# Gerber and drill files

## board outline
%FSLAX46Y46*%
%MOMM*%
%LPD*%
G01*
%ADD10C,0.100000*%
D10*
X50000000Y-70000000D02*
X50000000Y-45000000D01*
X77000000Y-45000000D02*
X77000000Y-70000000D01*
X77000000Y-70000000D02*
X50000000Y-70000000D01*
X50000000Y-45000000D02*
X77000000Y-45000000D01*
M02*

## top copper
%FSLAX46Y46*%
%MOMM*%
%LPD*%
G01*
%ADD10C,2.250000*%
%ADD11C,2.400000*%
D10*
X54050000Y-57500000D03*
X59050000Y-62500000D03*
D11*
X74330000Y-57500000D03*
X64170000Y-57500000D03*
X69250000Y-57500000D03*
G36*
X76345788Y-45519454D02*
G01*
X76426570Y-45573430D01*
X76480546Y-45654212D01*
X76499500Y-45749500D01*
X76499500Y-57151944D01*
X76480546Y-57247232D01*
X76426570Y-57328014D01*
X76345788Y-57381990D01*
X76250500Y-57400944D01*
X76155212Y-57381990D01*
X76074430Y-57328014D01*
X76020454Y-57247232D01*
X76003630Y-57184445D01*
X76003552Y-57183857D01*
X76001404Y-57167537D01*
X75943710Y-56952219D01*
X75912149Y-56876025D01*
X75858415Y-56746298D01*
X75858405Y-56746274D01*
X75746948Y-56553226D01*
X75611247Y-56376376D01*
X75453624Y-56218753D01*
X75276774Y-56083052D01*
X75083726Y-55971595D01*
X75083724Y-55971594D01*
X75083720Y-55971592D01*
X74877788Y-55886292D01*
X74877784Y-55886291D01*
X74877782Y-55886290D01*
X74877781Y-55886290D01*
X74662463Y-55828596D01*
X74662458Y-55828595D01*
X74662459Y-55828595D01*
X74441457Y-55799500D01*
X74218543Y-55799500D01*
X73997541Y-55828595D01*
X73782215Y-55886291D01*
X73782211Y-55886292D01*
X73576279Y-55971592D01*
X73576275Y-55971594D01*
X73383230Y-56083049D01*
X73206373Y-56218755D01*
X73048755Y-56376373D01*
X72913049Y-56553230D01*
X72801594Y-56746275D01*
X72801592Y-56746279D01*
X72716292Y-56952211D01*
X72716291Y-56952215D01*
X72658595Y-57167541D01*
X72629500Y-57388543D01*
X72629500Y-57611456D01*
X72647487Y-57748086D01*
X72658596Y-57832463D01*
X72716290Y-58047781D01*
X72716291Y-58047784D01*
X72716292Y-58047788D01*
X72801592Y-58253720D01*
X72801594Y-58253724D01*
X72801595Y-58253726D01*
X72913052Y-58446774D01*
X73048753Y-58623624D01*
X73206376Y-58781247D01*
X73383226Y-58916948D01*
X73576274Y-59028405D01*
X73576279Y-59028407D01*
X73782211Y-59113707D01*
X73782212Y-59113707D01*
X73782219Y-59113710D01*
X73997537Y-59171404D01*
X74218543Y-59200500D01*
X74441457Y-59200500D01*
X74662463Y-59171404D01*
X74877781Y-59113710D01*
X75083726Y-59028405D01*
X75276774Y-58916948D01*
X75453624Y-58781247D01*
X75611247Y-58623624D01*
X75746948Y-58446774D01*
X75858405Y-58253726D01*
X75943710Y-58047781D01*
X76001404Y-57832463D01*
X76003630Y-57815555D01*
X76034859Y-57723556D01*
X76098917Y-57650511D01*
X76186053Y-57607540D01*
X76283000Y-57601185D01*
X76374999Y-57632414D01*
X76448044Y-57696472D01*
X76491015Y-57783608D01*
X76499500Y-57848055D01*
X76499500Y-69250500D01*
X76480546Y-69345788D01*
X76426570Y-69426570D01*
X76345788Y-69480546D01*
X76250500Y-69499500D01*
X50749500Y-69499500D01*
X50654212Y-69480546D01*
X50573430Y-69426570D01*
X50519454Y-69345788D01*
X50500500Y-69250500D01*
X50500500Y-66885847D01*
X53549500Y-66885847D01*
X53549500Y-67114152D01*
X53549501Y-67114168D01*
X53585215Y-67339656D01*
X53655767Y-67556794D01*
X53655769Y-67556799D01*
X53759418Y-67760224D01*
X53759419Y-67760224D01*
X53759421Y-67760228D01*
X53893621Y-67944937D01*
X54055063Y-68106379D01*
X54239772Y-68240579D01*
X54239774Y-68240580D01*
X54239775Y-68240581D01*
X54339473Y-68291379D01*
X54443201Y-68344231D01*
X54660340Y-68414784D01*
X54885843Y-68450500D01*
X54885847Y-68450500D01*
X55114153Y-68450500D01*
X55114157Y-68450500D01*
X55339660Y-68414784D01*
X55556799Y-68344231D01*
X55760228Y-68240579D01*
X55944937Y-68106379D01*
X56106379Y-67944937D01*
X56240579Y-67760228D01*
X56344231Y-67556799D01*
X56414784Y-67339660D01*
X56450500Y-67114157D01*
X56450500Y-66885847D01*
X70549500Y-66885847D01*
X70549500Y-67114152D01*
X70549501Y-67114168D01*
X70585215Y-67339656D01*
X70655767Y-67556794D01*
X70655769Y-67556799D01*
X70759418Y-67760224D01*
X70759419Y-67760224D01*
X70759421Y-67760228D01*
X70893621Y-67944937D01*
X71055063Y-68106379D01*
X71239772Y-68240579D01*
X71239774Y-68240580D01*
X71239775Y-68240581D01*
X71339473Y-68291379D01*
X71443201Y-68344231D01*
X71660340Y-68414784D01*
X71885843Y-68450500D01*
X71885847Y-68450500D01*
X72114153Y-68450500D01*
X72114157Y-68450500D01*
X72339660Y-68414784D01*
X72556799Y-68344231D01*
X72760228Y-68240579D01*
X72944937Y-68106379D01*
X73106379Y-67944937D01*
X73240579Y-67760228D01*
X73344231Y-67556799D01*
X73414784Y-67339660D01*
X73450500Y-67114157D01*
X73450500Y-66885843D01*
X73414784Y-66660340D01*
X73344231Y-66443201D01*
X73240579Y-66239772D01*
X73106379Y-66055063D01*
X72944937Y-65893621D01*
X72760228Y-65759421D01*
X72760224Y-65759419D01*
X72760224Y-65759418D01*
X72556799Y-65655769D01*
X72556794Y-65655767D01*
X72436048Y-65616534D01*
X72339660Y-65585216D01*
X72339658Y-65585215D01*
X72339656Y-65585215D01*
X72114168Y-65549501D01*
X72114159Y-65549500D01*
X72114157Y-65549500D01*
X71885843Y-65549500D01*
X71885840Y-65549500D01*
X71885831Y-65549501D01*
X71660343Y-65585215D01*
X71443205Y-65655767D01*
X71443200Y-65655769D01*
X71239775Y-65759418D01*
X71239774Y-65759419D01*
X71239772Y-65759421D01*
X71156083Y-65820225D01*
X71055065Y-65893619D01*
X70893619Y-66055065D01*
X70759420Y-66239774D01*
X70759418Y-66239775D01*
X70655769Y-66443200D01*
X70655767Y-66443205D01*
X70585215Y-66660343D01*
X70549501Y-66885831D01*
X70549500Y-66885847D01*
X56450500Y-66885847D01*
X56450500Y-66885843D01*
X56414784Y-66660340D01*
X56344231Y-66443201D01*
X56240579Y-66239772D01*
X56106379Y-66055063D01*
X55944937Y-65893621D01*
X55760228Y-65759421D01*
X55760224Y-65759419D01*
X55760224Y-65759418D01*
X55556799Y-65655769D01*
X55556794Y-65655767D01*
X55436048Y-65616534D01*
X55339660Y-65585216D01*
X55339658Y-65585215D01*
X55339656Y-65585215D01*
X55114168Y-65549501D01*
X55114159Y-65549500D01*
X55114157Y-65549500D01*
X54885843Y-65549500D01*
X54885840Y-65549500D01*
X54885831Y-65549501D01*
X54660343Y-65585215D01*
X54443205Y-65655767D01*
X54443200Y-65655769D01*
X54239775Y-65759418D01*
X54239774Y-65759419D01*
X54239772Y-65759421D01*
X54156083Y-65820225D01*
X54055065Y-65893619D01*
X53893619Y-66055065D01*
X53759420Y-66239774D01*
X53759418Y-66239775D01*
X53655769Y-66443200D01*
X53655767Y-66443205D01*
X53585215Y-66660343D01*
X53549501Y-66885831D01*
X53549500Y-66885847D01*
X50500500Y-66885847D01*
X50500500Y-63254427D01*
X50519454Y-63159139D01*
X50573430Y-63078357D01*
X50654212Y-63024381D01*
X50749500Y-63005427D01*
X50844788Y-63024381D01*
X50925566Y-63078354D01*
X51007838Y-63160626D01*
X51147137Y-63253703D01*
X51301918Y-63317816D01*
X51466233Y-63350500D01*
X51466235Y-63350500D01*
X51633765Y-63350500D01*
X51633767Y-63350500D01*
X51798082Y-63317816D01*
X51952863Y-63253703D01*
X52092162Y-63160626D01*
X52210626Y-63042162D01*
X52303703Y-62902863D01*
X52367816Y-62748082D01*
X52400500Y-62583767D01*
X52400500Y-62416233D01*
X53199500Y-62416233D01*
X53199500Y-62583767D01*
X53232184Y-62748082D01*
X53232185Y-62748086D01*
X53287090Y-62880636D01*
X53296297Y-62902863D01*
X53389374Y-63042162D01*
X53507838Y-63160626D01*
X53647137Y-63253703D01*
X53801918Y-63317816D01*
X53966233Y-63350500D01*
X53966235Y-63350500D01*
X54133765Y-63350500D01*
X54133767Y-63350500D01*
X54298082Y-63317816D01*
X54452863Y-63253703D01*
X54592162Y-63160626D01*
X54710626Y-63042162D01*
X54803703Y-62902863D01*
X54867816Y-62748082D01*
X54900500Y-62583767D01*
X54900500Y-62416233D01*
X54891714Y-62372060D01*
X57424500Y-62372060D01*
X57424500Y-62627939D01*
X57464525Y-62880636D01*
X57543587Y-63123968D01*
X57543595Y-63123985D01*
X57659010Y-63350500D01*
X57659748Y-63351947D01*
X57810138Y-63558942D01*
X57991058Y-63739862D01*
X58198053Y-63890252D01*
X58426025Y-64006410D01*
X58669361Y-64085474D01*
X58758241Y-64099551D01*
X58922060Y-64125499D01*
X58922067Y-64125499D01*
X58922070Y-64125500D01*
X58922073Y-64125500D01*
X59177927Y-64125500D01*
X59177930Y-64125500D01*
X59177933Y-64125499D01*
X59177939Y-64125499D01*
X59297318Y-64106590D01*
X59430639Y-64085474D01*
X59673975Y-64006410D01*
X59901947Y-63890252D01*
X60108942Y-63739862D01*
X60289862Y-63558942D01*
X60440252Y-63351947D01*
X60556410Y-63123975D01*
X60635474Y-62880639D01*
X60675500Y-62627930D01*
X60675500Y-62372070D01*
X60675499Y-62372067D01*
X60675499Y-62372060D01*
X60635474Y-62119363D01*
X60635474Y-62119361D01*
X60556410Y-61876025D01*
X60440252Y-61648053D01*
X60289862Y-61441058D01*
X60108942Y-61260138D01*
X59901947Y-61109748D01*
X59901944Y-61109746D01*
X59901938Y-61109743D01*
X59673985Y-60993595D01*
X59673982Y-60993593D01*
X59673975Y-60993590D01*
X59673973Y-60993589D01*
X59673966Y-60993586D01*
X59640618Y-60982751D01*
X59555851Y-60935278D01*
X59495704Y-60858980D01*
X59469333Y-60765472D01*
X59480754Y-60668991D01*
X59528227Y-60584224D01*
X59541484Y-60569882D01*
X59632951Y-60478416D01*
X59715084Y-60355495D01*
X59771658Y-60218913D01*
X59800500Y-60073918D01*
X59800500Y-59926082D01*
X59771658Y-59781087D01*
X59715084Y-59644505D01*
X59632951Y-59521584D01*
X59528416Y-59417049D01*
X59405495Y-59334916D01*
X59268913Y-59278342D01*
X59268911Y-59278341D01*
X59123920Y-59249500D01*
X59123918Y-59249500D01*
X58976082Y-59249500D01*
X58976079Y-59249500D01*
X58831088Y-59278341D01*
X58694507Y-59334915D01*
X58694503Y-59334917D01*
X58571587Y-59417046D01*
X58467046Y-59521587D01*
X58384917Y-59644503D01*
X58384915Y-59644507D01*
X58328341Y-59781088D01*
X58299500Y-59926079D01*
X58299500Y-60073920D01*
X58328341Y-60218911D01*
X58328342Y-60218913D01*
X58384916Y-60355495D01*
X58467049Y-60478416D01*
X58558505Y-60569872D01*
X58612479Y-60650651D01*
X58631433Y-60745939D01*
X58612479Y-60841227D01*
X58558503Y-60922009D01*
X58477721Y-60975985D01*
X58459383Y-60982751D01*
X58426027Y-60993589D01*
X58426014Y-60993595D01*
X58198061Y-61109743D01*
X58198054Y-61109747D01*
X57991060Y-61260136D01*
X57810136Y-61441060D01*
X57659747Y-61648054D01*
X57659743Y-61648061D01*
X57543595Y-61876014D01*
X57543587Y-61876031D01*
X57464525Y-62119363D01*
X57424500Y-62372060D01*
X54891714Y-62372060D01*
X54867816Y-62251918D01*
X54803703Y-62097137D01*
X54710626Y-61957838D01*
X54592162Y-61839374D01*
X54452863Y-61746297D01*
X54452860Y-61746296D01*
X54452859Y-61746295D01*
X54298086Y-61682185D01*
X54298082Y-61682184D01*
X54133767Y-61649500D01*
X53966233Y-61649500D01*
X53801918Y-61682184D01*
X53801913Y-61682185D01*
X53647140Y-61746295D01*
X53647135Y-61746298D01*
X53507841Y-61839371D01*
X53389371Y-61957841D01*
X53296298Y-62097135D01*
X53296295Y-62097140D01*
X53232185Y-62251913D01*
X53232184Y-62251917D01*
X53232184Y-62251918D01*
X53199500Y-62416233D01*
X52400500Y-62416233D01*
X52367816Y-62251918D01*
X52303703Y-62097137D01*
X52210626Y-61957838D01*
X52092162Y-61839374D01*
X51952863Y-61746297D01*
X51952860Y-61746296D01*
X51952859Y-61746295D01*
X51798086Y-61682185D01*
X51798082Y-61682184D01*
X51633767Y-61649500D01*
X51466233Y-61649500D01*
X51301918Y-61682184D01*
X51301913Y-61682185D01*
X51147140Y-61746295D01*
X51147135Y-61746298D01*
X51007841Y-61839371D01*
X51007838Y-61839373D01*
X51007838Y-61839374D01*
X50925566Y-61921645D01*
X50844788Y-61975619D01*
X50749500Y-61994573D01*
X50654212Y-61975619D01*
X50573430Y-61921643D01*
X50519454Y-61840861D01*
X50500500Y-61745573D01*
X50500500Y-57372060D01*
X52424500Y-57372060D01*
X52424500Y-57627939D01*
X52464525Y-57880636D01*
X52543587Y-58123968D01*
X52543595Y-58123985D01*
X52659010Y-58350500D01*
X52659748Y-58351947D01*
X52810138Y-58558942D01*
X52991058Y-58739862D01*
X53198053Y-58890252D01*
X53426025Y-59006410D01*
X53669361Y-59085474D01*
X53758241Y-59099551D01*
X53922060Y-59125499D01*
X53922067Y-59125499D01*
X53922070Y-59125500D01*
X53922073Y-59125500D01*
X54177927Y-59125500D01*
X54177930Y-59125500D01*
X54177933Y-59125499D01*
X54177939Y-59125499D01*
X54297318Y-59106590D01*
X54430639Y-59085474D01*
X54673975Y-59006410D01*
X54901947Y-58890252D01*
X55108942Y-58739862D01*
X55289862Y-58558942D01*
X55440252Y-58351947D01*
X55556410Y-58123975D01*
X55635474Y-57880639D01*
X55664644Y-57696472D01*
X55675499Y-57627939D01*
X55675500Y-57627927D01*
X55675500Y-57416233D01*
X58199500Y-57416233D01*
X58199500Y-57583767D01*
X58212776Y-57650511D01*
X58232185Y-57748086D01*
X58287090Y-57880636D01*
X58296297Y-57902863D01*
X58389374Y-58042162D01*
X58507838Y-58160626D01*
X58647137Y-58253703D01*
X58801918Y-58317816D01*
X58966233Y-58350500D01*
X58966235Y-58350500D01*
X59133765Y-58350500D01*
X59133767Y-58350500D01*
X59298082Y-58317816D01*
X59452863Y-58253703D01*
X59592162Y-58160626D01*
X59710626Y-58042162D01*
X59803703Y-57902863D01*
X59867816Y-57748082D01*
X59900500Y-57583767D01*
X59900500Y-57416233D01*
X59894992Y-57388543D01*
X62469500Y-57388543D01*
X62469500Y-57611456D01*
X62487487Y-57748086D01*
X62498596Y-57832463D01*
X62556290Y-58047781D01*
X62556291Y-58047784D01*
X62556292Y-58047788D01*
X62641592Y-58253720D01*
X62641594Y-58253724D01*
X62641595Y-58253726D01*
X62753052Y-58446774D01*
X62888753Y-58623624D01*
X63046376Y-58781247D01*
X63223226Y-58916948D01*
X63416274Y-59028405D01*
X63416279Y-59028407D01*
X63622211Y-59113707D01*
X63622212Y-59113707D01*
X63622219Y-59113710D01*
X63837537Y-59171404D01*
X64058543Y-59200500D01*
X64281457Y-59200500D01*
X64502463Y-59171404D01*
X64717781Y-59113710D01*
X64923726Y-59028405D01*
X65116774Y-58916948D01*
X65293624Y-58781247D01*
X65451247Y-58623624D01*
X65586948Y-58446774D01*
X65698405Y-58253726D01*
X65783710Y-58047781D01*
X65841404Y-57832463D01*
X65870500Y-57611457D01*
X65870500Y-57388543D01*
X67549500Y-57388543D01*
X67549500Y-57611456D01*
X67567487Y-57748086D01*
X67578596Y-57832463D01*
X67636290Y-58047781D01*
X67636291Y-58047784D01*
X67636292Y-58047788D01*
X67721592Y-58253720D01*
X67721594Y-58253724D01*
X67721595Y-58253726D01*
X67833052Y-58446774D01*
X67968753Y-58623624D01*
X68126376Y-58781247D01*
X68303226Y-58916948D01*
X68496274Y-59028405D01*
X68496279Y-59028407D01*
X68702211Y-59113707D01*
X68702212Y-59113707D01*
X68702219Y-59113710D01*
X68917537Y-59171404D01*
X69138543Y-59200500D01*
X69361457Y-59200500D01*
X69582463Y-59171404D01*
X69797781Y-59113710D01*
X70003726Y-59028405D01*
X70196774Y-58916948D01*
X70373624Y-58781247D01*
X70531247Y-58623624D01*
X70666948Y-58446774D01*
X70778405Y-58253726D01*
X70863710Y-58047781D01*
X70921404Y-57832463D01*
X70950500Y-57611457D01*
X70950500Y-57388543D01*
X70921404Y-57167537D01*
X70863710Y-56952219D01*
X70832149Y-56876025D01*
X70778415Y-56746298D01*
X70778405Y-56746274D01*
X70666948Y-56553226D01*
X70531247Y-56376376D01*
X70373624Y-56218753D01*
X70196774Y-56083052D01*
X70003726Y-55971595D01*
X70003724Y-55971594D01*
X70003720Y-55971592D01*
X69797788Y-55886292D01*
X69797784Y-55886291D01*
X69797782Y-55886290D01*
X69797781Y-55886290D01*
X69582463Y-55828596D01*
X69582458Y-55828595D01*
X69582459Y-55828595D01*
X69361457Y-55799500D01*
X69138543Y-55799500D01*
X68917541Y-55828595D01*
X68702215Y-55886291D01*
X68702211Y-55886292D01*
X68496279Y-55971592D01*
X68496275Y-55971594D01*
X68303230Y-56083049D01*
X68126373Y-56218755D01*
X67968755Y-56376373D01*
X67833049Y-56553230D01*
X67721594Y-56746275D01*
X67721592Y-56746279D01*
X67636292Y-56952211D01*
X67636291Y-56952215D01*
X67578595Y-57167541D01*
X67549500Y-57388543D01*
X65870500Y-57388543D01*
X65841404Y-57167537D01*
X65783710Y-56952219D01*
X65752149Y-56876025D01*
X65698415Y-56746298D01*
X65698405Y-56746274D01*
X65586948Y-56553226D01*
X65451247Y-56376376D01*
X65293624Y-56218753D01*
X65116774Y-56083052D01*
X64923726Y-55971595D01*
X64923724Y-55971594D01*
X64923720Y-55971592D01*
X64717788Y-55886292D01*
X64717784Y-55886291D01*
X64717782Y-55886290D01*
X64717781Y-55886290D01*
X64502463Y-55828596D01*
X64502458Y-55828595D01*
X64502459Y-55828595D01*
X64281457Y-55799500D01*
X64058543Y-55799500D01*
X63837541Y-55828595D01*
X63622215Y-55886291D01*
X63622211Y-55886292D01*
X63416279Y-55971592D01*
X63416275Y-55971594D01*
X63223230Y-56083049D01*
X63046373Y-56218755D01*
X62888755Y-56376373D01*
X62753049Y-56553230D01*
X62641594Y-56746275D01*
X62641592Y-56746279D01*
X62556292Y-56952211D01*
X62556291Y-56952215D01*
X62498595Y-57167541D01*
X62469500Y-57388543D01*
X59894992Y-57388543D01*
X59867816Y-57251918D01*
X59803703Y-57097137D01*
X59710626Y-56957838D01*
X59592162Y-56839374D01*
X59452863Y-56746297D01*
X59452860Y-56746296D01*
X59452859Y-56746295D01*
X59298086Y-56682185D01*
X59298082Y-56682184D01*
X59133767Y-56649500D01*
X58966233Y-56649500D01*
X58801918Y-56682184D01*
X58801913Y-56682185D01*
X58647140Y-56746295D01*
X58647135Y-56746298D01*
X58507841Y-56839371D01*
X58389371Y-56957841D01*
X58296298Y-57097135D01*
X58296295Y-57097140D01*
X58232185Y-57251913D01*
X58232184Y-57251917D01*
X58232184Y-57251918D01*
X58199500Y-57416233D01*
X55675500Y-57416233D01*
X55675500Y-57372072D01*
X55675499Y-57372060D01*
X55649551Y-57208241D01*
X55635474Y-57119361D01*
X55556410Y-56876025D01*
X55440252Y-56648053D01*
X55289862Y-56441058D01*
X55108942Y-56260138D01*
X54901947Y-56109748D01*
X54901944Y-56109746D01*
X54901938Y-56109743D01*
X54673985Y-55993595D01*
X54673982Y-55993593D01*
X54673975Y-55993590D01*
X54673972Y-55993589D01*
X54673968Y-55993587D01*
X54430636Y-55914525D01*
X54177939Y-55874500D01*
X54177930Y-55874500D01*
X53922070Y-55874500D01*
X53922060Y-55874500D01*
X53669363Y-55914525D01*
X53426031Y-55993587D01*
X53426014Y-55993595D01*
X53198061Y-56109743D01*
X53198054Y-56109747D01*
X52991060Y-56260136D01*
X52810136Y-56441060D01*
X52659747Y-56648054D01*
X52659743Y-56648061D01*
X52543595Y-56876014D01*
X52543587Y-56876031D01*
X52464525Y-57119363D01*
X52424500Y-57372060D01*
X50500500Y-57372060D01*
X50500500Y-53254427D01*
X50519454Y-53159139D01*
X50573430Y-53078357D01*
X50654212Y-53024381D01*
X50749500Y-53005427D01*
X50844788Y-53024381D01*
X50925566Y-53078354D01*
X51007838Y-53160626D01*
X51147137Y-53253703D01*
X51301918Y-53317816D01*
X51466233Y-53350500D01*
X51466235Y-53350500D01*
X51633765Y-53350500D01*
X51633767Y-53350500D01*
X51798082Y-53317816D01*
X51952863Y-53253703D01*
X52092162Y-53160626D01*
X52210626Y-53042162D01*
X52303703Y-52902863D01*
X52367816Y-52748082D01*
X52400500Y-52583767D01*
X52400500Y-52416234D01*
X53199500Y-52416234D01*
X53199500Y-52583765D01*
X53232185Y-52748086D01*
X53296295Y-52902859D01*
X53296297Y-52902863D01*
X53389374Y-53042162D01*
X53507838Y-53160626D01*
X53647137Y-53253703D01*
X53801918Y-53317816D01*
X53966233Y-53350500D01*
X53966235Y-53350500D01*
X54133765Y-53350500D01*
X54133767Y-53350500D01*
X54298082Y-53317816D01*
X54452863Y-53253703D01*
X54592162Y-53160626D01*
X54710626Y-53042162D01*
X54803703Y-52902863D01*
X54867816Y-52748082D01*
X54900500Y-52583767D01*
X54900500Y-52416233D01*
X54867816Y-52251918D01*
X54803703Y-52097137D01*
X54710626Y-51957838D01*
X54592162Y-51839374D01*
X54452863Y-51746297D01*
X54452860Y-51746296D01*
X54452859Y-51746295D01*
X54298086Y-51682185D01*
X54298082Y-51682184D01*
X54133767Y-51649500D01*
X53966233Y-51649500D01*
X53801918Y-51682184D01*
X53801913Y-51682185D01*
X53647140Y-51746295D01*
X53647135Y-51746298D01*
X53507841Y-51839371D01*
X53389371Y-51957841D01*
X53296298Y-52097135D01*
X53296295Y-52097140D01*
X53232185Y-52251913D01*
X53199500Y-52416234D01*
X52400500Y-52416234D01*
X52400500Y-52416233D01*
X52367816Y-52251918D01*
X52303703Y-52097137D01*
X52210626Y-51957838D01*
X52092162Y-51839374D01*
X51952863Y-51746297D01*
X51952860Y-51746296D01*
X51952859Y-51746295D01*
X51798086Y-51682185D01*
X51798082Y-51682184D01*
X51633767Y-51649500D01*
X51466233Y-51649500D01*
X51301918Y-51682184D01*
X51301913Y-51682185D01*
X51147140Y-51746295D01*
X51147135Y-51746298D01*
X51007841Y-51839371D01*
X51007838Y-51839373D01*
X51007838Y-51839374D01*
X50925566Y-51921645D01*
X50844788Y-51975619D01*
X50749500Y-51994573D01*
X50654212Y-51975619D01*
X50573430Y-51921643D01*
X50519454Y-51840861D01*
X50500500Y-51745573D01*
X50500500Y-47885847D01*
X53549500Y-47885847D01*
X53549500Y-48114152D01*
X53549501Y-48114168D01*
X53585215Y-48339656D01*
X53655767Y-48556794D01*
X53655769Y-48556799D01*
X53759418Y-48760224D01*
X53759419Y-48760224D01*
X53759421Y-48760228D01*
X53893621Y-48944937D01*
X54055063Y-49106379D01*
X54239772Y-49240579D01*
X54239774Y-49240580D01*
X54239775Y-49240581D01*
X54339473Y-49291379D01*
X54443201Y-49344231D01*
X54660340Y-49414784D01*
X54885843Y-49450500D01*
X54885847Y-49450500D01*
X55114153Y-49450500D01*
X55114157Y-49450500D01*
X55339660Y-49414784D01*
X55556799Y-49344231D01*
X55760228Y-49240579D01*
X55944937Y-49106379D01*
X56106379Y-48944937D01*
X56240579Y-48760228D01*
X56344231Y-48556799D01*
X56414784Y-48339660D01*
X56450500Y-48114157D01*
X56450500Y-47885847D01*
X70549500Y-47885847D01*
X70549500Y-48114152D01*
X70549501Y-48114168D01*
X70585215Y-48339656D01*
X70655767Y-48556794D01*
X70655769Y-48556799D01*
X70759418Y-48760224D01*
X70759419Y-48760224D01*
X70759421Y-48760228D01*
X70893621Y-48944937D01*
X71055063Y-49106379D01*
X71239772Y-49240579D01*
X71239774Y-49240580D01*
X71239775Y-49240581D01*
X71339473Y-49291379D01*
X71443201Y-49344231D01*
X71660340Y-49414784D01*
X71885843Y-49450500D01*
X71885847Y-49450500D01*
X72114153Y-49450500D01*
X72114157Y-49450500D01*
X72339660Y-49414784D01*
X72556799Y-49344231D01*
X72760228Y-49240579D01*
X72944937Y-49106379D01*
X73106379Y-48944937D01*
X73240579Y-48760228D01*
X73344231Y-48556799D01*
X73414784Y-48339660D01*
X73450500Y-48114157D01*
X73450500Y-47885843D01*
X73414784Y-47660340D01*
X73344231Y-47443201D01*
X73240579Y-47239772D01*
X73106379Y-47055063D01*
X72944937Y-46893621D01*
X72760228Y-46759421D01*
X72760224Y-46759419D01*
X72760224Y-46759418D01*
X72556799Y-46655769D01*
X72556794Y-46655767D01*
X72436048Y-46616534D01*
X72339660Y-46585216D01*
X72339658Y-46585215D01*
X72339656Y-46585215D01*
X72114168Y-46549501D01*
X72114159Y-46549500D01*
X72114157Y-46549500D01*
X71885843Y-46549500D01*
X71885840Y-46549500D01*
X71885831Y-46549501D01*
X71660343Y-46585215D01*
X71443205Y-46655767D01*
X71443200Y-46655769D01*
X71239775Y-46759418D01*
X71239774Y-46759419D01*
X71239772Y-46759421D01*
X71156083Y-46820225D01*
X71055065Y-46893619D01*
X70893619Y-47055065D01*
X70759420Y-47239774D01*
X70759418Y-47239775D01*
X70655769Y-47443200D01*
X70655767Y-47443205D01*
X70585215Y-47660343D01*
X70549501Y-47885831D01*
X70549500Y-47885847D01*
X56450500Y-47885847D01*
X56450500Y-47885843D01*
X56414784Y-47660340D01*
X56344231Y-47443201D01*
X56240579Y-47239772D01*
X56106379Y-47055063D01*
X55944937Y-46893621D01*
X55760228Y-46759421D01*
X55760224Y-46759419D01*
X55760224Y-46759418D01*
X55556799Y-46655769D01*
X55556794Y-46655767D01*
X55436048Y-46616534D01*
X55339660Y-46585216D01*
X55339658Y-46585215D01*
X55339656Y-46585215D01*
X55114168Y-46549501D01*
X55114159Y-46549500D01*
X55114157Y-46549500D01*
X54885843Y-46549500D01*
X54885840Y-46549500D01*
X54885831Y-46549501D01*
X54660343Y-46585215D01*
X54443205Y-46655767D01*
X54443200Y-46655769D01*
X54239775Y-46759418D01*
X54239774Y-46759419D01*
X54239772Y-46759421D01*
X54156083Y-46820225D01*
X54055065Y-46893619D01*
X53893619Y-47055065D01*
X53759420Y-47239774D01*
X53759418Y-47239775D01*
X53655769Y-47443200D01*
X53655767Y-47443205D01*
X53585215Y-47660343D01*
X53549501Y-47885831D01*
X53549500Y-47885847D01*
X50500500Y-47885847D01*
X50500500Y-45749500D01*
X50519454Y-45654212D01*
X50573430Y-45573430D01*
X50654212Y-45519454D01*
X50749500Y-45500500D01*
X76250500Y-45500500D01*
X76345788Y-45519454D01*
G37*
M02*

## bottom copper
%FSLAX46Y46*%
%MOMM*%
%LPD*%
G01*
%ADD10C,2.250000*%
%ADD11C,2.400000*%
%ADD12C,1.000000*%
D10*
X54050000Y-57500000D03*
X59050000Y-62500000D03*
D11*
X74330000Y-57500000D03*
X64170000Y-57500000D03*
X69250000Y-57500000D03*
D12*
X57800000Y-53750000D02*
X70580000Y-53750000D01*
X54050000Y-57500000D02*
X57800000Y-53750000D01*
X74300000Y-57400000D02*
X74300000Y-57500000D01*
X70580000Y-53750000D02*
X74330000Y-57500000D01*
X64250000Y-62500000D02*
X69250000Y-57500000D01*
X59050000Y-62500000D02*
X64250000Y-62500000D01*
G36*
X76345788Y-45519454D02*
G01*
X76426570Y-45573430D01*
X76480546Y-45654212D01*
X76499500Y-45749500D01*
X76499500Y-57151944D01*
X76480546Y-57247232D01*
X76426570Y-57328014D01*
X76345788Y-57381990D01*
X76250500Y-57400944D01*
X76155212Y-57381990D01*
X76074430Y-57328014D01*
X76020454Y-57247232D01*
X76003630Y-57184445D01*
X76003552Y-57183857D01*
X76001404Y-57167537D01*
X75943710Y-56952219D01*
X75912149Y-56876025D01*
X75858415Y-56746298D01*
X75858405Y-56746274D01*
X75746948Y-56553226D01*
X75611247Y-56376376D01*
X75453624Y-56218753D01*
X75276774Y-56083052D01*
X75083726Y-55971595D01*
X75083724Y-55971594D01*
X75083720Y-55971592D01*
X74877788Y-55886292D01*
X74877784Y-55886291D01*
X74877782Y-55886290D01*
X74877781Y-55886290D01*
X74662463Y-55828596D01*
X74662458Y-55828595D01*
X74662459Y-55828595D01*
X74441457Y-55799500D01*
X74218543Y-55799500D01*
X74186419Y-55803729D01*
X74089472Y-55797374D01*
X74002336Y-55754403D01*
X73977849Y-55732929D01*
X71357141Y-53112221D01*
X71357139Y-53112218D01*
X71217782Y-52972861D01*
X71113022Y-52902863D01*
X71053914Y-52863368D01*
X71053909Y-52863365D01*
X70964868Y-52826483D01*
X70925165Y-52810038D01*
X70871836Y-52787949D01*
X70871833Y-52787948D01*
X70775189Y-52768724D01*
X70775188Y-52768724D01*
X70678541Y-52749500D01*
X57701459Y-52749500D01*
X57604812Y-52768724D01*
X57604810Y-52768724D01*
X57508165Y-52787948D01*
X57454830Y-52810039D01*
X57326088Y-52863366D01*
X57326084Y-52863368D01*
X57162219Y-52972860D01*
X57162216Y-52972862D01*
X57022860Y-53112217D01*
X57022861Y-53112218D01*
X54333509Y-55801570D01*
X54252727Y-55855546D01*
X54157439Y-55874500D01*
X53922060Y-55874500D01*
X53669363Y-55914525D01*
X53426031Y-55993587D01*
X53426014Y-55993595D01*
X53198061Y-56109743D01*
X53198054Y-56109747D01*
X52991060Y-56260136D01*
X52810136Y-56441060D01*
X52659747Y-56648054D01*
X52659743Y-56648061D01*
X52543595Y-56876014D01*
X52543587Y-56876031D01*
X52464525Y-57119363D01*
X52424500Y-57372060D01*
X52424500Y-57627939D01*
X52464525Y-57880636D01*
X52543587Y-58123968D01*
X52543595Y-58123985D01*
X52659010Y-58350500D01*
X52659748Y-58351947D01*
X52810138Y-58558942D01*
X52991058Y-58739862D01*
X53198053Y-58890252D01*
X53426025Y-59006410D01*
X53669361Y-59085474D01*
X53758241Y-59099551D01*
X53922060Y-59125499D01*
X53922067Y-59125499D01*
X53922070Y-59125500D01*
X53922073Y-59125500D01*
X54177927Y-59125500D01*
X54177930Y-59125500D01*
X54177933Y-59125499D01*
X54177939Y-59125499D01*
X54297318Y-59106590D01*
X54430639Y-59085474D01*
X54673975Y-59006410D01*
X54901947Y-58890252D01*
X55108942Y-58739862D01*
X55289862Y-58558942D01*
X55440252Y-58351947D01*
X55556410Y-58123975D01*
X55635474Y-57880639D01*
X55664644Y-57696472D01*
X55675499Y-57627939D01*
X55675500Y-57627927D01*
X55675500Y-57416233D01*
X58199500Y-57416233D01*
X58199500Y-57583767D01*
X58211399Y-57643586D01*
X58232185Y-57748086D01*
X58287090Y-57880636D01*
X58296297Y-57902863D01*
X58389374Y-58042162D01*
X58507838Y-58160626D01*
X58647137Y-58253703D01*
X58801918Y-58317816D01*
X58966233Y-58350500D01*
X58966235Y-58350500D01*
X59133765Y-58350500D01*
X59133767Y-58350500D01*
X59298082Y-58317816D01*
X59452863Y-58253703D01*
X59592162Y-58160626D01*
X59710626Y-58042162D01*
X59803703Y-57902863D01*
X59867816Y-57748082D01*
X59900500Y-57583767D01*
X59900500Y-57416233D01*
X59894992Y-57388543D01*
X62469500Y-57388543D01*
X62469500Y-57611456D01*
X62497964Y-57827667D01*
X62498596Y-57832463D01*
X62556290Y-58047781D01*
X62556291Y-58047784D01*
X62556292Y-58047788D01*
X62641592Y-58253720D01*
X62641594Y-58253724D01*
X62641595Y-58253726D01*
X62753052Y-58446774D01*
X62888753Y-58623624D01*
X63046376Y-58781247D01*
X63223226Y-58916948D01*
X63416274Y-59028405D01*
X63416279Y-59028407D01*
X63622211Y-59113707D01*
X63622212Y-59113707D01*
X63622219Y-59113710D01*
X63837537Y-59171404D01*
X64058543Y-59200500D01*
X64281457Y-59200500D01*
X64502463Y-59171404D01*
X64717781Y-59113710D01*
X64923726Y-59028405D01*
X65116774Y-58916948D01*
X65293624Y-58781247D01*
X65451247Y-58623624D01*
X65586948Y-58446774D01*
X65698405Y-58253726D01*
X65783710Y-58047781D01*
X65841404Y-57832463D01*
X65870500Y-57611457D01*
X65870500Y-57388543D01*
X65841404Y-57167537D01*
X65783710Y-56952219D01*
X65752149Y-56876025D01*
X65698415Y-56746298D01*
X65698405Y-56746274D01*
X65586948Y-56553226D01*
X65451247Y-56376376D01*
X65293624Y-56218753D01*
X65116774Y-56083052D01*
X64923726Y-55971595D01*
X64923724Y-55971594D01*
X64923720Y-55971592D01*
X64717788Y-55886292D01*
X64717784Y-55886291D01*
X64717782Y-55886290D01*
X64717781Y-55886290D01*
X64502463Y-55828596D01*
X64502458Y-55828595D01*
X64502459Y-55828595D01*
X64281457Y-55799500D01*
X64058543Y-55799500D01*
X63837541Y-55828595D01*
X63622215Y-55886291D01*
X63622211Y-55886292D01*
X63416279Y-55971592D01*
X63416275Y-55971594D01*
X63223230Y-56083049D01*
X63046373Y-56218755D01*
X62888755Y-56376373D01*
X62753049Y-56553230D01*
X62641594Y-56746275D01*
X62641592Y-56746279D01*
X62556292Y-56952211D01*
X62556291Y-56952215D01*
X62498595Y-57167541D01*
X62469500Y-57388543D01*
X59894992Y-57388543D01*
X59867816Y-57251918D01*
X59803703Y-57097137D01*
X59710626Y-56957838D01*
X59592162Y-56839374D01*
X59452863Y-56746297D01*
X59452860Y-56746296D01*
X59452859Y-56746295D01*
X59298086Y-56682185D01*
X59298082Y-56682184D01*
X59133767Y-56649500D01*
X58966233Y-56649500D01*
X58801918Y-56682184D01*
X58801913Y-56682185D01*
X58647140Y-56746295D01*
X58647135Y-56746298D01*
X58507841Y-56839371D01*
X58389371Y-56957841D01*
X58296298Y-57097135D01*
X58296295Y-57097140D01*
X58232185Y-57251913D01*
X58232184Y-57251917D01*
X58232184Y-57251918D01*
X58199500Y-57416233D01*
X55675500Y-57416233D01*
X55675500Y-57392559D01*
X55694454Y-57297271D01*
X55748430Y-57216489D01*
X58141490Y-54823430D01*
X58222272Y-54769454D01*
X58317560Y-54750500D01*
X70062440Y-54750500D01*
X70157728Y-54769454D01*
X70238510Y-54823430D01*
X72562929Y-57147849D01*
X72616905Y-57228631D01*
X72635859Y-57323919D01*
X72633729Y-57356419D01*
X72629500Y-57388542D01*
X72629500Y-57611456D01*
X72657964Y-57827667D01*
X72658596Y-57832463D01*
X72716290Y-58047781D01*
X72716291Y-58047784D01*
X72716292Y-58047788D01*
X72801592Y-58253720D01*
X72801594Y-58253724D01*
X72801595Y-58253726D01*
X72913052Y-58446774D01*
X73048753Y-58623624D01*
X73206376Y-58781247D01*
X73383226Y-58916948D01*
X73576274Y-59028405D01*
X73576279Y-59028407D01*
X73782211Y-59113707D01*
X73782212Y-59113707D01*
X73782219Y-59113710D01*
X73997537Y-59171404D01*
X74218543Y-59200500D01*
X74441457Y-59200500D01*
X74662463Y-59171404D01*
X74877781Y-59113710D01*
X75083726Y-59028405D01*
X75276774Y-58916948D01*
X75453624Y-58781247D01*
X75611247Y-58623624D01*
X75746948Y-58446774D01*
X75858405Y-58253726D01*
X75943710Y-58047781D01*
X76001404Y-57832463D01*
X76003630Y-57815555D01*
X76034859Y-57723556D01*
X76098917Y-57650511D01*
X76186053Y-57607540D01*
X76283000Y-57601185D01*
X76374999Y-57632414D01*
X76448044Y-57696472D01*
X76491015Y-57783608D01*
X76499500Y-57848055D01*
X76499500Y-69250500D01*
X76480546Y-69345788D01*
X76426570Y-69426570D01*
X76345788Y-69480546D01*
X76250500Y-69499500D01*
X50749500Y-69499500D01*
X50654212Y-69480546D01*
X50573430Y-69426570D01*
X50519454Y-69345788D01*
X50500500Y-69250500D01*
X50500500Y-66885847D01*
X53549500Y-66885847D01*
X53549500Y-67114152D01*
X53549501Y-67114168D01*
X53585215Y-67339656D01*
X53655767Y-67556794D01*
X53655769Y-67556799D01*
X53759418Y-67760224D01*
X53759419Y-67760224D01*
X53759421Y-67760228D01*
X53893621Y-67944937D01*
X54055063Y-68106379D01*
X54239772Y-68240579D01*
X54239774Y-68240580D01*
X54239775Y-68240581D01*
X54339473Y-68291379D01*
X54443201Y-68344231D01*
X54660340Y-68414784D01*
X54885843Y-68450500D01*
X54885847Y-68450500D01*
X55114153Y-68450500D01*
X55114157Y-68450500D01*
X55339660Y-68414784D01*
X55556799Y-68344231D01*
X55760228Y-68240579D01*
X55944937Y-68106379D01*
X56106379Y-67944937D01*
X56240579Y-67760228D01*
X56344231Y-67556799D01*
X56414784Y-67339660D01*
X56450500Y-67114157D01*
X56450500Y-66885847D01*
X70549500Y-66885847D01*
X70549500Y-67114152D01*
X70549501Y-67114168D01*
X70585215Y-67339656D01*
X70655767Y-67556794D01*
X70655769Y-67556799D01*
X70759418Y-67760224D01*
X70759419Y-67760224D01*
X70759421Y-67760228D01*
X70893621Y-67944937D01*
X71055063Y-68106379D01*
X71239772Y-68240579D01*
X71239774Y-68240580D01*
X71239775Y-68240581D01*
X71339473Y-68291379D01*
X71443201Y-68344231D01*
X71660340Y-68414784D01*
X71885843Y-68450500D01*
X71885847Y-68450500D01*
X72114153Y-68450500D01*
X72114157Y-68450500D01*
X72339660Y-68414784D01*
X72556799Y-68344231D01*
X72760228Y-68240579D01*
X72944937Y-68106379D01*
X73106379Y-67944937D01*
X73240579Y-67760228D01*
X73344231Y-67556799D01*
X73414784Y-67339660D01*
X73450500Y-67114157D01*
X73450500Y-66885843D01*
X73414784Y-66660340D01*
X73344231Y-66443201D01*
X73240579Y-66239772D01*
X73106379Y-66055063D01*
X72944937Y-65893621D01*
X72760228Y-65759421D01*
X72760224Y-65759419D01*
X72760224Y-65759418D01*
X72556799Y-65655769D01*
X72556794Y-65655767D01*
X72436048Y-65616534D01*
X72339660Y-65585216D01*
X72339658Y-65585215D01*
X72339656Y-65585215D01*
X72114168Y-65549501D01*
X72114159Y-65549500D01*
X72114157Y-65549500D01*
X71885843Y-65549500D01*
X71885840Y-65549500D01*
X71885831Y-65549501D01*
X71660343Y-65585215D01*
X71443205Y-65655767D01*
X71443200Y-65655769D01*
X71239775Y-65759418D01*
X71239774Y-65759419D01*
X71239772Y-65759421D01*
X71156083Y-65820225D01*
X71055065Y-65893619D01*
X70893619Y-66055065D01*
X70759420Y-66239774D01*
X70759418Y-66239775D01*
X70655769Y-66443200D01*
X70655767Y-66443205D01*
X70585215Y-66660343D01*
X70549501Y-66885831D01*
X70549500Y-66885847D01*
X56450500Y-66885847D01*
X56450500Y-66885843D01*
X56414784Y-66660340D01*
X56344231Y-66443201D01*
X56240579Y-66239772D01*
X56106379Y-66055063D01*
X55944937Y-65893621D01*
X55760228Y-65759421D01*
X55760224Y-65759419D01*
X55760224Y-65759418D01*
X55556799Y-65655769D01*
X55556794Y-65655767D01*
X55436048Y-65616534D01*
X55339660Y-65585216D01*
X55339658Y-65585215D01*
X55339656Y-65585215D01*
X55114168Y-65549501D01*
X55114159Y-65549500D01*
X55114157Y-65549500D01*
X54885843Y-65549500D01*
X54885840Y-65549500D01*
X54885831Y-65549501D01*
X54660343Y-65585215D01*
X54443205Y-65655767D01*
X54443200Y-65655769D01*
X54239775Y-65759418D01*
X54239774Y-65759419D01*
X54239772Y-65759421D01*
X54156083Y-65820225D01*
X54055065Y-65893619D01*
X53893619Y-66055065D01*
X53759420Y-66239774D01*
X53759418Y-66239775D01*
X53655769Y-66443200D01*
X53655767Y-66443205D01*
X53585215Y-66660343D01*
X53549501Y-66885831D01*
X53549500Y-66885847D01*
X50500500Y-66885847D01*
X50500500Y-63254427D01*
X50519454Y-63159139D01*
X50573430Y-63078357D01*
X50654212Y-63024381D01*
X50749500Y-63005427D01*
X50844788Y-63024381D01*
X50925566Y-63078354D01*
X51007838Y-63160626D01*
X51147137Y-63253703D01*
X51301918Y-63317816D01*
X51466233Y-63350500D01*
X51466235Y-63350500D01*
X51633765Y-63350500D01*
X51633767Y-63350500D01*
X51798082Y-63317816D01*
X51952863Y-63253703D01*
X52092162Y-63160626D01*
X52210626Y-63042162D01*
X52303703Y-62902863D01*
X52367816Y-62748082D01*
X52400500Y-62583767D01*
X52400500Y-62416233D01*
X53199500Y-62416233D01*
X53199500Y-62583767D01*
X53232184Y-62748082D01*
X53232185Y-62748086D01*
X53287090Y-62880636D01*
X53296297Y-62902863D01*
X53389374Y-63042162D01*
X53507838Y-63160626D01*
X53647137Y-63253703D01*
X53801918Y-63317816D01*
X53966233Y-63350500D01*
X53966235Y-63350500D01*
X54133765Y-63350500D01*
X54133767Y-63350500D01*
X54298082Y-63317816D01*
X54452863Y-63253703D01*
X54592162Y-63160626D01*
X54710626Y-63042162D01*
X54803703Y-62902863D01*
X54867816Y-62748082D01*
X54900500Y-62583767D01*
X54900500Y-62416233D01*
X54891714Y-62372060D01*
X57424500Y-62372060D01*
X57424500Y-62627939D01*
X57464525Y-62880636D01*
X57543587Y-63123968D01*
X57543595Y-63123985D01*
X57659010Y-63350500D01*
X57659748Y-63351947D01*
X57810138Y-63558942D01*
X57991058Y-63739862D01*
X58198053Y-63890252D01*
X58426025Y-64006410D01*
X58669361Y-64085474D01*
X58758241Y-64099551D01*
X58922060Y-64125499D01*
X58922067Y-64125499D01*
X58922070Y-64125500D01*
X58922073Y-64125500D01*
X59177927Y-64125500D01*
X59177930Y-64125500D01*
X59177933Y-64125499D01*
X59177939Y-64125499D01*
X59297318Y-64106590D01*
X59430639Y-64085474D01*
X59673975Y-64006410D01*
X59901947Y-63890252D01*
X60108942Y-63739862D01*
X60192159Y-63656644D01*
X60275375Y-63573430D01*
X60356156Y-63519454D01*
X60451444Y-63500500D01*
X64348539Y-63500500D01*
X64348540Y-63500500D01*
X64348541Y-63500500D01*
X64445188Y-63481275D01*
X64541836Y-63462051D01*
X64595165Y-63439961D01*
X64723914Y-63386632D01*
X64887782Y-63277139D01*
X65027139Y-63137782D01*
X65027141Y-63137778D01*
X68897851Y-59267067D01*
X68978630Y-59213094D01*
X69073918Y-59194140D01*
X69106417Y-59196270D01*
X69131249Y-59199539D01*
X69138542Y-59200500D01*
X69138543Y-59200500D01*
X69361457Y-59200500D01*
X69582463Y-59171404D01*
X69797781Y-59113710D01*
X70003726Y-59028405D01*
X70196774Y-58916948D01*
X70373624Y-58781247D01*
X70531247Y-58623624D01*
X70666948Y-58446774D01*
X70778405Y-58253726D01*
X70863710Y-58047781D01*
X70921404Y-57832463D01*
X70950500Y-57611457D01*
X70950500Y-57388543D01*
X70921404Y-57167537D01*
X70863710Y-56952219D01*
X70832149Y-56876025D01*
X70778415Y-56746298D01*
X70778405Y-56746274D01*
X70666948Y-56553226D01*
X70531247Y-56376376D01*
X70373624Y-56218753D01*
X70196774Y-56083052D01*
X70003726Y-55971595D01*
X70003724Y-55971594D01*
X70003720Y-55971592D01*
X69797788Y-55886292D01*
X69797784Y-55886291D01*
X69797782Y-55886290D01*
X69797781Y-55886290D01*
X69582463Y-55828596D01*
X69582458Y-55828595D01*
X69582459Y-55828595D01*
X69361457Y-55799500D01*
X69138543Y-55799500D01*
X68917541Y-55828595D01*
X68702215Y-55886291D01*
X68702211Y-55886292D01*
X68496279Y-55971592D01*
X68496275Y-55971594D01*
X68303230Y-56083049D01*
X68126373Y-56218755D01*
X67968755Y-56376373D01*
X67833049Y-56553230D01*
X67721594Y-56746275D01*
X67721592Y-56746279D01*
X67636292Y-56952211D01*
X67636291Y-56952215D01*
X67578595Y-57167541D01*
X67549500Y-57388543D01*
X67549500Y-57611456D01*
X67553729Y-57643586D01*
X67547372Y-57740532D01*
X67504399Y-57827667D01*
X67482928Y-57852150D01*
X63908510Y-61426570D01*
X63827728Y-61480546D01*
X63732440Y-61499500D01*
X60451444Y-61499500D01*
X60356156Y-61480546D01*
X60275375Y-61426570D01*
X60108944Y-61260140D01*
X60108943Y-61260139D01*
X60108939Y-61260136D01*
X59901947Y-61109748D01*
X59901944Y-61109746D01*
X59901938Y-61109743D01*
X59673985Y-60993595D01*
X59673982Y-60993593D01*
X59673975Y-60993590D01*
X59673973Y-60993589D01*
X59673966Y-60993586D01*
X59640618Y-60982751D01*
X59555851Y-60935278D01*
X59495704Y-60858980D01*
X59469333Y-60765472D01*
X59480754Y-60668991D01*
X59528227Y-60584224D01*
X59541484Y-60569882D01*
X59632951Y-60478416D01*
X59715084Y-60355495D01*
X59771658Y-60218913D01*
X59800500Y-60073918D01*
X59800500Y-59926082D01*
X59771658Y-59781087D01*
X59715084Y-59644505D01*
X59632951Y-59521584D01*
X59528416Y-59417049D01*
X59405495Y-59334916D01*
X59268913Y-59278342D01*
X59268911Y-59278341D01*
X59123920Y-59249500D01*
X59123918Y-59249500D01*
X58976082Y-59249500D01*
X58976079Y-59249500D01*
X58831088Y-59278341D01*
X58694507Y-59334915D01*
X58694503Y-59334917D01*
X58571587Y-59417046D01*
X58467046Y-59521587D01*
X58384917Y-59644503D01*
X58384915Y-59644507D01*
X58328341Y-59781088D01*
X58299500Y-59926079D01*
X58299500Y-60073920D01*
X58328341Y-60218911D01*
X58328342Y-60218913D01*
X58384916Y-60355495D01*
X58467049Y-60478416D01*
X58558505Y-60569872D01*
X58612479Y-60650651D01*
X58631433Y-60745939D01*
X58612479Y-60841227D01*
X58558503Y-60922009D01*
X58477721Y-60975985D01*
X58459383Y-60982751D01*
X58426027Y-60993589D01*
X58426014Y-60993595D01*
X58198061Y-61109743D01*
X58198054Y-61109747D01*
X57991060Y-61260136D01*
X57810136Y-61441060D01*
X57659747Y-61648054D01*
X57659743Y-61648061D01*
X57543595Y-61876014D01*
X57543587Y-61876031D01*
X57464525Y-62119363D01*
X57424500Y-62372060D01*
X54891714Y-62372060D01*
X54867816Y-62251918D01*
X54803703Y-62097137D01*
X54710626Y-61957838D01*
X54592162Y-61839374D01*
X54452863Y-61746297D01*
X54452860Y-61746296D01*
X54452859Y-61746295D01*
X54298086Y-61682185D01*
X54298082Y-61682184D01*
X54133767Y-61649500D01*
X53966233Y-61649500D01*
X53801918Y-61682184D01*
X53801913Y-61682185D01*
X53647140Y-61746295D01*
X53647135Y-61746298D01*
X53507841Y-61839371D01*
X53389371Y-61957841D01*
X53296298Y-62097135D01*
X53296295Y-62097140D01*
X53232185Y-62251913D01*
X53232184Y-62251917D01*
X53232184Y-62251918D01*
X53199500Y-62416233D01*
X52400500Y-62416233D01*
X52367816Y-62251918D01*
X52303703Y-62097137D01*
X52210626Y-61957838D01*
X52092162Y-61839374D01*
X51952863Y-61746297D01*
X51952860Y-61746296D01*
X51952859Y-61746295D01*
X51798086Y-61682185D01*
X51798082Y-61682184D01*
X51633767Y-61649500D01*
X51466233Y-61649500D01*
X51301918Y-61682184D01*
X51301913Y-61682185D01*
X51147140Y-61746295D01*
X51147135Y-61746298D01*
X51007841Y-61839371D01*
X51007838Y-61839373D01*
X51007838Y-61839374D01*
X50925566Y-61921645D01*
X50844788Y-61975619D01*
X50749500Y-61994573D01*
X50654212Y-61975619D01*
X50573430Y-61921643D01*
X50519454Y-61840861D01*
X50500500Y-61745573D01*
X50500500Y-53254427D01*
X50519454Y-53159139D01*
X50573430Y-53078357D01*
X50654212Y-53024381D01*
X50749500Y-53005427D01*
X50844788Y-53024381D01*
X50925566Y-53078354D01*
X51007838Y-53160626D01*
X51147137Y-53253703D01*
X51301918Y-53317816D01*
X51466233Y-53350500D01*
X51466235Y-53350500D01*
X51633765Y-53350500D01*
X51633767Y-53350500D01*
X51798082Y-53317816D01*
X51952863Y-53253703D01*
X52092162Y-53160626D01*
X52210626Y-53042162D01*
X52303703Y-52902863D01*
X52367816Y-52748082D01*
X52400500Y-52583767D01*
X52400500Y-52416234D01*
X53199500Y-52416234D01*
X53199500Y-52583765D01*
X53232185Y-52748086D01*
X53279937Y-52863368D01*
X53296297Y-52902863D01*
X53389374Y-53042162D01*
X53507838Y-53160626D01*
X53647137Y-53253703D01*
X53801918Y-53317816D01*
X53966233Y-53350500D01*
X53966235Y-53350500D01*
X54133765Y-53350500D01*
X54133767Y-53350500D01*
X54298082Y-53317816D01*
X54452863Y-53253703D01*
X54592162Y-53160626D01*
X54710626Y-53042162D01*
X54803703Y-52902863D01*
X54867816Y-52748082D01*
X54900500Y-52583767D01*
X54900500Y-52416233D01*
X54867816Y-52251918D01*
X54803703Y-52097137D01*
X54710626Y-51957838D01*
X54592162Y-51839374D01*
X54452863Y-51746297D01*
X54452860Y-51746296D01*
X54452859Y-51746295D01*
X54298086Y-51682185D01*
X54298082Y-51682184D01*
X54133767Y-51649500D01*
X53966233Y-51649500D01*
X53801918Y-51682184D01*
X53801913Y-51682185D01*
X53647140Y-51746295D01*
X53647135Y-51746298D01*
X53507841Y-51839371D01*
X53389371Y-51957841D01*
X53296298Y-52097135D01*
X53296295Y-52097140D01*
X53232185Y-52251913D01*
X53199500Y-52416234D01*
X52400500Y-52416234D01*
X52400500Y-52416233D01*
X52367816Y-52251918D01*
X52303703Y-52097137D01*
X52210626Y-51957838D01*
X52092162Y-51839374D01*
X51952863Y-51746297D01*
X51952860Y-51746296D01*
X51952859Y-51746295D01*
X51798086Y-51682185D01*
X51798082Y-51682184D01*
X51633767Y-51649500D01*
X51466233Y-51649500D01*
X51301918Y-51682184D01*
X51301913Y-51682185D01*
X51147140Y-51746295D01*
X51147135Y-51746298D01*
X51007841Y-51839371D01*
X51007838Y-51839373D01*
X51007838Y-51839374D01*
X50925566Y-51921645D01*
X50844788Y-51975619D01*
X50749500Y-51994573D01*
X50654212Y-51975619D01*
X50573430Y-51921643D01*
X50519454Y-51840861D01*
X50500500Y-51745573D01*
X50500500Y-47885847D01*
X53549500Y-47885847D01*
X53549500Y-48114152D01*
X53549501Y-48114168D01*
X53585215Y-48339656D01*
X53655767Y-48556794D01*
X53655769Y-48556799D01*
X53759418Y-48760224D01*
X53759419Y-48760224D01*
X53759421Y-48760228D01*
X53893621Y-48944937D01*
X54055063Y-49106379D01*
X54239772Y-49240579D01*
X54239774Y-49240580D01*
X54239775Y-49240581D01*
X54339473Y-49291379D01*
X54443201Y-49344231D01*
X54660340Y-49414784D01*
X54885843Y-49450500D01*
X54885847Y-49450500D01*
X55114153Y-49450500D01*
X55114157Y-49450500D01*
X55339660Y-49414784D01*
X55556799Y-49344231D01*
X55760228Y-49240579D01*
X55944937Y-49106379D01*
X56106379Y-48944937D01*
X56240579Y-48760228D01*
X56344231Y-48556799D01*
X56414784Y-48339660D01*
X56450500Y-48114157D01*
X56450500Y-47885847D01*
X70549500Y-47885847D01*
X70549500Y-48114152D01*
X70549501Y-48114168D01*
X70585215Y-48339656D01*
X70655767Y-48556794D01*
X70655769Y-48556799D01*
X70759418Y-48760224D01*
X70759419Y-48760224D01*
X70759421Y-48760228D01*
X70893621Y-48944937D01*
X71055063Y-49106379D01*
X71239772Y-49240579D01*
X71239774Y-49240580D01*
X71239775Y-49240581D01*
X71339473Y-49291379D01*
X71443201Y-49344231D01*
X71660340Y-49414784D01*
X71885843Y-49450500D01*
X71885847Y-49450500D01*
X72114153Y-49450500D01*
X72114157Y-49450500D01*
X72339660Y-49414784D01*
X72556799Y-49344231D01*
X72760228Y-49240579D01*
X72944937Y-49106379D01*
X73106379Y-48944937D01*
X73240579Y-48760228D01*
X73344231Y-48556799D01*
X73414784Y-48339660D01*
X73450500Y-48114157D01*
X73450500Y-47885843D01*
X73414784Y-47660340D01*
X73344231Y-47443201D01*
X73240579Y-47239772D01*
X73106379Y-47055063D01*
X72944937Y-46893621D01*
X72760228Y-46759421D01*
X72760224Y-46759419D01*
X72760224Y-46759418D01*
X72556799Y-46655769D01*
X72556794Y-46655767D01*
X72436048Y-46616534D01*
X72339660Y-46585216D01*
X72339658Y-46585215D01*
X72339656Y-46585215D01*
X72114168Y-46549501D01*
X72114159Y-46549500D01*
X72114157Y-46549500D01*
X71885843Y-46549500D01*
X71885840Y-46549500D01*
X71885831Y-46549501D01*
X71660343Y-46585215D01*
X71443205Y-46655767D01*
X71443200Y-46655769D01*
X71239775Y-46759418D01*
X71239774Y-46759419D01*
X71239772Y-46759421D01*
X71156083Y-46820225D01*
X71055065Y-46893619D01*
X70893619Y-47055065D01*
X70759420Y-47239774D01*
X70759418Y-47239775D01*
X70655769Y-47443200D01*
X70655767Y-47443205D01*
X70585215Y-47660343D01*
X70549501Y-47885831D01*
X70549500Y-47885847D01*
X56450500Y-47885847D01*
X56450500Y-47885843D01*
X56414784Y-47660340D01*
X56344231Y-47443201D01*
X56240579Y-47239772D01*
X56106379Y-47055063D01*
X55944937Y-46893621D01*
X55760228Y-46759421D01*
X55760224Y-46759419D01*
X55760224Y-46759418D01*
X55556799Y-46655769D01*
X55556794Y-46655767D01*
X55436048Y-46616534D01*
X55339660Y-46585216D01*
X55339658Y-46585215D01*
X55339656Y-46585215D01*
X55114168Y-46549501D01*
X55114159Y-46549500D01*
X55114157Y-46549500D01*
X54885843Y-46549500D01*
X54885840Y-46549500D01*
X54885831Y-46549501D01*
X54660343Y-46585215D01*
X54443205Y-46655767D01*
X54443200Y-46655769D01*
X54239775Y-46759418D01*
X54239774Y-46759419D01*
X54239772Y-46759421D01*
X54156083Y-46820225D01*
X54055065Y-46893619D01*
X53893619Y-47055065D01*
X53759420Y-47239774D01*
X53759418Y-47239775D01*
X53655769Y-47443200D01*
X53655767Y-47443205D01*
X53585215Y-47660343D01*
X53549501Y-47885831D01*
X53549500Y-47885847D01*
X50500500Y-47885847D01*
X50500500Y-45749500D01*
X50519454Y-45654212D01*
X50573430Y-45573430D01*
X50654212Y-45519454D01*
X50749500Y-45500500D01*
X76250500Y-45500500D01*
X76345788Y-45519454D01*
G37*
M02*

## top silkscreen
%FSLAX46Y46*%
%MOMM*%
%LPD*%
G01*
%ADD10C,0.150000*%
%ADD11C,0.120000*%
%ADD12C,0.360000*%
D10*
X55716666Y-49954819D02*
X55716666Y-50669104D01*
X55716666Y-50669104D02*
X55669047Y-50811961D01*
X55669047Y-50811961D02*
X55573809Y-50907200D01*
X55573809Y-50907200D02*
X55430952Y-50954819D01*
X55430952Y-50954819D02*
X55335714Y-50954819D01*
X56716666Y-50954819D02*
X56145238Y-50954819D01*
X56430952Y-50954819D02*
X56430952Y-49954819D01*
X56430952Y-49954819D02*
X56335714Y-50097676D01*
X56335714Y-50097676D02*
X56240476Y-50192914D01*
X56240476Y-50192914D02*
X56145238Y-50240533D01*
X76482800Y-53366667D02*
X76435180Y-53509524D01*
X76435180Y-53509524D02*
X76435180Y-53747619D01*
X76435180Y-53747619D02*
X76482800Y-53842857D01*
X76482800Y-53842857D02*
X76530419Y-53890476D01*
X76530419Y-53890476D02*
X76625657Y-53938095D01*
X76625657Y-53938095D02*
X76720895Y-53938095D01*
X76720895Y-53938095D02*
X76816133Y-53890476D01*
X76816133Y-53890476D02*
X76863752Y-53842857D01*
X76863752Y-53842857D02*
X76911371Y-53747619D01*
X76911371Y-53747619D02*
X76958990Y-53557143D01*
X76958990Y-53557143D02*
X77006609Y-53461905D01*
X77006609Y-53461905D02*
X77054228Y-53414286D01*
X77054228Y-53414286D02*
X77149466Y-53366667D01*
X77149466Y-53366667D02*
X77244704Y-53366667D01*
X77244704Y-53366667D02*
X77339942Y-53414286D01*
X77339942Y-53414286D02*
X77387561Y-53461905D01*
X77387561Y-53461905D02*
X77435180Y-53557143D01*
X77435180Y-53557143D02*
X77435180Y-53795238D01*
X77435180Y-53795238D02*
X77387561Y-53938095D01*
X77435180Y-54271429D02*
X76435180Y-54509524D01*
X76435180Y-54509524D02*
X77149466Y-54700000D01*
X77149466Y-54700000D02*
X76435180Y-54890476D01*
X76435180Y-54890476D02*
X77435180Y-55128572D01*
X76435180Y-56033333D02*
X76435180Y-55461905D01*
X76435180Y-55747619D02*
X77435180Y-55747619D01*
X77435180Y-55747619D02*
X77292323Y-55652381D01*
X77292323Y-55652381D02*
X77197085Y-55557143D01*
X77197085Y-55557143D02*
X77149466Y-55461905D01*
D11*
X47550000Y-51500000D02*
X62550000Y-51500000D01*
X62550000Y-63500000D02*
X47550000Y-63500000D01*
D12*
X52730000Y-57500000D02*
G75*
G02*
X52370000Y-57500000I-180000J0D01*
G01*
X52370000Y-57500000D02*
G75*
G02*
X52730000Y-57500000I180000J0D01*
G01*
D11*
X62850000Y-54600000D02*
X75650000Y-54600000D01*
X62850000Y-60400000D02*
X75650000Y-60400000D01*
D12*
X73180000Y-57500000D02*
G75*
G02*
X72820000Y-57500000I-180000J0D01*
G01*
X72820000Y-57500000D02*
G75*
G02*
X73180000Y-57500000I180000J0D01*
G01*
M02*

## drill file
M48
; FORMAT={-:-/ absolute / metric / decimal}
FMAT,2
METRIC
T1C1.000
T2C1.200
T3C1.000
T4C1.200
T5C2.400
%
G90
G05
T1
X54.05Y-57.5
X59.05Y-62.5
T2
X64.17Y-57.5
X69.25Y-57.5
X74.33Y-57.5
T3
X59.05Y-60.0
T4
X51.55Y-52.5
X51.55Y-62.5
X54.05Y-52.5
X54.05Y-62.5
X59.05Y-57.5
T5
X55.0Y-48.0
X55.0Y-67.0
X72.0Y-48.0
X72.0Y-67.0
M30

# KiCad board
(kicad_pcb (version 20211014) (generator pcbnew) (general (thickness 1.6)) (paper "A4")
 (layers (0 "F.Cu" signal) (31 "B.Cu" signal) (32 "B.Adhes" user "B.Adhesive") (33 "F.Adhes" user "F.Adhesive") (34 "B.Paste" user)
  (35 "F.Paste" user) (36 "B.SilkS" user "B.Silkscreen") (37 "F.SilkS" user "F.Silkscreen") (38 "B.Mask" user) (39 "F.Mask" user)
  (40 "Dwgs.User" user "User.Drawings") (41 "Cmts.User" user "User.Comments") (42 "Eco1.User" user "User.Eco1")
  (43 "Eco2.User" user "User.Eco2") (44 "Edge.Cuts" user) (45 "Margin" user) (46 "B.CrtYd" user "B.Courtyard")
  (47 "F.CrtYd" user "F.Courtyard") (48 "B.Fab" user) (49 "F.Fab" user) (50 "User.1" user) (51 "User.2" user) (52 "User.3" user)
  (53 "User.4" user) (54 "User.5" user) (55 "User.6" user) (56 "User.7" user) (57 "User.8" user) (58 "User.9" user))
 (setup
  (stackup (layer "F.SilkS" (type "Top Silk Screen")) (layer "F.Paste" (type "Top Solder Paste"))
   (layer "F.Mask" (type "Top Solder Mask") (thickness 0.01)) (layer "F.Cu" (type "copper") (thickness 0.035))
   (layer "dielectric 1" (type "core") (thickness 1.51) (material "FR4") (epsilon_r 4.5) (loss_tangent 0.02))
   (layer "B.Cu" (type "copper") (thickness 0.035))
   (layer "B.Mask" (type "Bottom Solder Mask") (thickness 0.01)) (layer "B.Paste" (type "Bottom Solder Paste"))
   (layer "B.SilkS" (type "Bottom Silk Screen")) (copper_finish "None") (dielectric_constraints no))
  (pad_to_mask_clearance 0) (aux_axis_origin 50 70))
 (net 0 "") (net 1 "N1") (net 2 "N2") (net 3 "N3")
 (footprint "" (layer "F.Cu") (at 73.06 67.12)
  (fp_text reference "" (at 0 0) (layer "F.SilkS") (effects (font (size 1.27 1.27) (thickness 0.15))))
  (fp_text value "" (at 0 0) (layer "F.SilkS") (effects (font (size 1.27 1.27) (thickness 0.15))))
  (pad "" np_thru_hole circle (at -1.06 -0.12) (size 2.4 2.4) (drill 2.4) (layers F&B.Cu *.Mask)))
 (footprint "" (layer "F.Cu") (at 53 48)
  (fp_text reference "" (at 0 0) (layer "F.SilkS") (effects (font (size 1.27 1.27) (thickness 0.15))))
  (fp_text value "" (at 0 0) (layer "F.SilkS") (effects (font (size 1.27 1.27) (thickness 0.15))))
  (pad "" np_thru_hole circle (at 2 0) (size 2.4 2.4) (drill 2.4) (layers F&B.Cu *.Mask)))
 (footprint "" (layer "F.Cu") (at 72 47.5)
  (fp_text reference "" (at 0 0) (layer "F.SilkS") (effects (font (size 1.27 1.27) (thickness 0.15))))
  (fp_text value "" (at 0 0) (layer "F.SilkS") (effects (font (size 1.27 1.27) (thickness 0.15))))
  (pad "" np_thru_hole circle (at 0 0.5) (size 2.4 2.4) (drill 2.4) (layers F&B.Cu *.Mask)))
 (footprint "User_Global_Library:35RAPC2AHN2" (layer "F.Cu") (at 55.05 57.5)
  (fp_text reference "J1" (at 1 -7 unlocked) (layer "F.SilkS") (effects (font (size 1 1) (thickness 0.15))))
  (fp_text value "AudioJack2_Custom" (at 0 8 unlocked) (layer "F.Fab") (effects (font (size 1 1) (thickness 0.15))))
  (fp_line (start -7.5 -6) (end 7.5 -6) (layer "F.SilkS") (width 0.12))
  (fp_line (start 7.5 6) (end -7.5 6) (layer "F.SilkS") (width 0.12))
  (fp_circle (center -2.5 0) (end -2.2 0) (layer "F.SilkS") (width 0.12) (fill solid))
  (pad "" np_thru_hole circle (at -3.5 5) (size 1.2 1.2) (drill 1.2) (layers F&B.Cu *.Mask))
  (pad "" np_thru_hole circle (at -1 5) (size 1.2 1.2) (drill 1.2) (layers F&B.Cu *.Mask))
  (pad "" np_thru_hole circle (at 4 0) (size 1.2 1.2) (drill 1.2) (layers F&B.Cu *.Mask))
  (pad "" np_thru_hole circle (at -3.5 -5) (size 1.2 1.2) (drill 1.2) (layers F&B.Cu *.Mask))
  (pad "" np_thru_hole circle (at 4 2.5) (size 1 1) (drill 1) (layers F&B.Cu *.Mask))
  (pad "" np_thru_hole circle (at -1 -5) (size 1.2 1.2) (drill 1.2) (layers F&B.Cu *.Mask))
  (pad "S" thru_hole circle (at -1 0) (size 2.25 2.25) (drill 1) (layers *.Cu *.Mask) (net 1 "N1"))
  (pad "T" thru_hole circle (at 4 5) (size 2.25 2.25) (drill 1) (layers *.Cu *.Mask) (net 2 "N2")))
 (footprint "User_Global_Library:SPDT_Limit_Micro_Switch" (layer "F.Cu") (at 69.25 57.5)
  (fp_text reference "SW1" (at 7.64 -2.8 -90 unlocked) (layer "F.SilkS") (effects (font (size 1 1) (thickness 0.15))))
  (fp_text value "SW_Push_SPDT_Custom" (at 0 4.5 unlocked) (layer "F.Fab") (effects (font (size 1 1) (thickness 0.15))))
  (fp_line (start -6.4 -2.9) (end 6.4 -2.9) (layer "F.SilkS") (width 0.12))
  (fp_line (start -6.4 2.9) (end 6.4 2.9) (layer "F.SilkS") (width 0.12))
  (fp_circle (center 3.75 0) (end 4.05 0) (layer "F.SilkS") (width 0.12) (fill solid))
  (pad "1" thru_hole circle (at 5.08 0) (size 2.4 2.4) (drill 1.2) (layers *.Cu *.Mask) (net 1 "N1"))
  (pad "2" thru_hole circle (at -5.08 0) (size 2.4 2.4) (drill 1.2) (layers *.Cu *.Mask) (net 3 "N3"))
  (pad "3" thru_hole circle (at 0 0) (size 2.4 2.4) (drill 1.2) (layers *.Cu *.Mask) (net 2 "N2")))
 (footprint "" (layer "F.Cu") (at 53 67)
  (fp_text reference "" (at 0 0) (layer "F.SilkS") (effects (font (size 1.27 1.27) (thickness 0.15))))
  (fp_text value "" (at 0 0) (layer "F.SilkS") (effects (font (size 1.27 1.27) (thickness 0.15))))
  (pad "" np_thru_hole circle (at 2 0) (size 2.4 2.4) (drill 2.4) (layers F&B.Cu *.Mask)))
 (gr_line (start 50 70) (end 50 45) (layer "Edge.Cuts") (width 0.1))
 (gr_line (start 77 45) (end 77 70) (layer "Edge.Cuts") (width 0.1))
 (gr_line (start 77 70) (end 50 70) (layer "Edge.Cuts") (width 0.1))
 (gr_line (start 50 45) (end 77 45) (layer "Edge.Cuts") (width 0.1))
 (segment (start 57.8 53.75) (end 70.58 53.75) (width 1) (layer "B.Cu") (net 1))
 (segment (start 54.05 57.5) (end 57.8 53.75) (width 1) (layer "B.Cu") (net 1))
 (segment (start 74.3 57.4) (end 74.3 57.5) (width 1) (layer "B.Cu") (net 1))
 (segment (start 70.58 53.75) (end 74.33 57.5) (width 1) (layer "B.Cu") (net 1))
 (segment (start 64.25 62.5) (end 69.25 57.5) (width 1) (layer "B.Cu") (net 2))
 (segment (start 59.05 62.5) (end 64.25 62.5) (width 1) (layer "B.Cu") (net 2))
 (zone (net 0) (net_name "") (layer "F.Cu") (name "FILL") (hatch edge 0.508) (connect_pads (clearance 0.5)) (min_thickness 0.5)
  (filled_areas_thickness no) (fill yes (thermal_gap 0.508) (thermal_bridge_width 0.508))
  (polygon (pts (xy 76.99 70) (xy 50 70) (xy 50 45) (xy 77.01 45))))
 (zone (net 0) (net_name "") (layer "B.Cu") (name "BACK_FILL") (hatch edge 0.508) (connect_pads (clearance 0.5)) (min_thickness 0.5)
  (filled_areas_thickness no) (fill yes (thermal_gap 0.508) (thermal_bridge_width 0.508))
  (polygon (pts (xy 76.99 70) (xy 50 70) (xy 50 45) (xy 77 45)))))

